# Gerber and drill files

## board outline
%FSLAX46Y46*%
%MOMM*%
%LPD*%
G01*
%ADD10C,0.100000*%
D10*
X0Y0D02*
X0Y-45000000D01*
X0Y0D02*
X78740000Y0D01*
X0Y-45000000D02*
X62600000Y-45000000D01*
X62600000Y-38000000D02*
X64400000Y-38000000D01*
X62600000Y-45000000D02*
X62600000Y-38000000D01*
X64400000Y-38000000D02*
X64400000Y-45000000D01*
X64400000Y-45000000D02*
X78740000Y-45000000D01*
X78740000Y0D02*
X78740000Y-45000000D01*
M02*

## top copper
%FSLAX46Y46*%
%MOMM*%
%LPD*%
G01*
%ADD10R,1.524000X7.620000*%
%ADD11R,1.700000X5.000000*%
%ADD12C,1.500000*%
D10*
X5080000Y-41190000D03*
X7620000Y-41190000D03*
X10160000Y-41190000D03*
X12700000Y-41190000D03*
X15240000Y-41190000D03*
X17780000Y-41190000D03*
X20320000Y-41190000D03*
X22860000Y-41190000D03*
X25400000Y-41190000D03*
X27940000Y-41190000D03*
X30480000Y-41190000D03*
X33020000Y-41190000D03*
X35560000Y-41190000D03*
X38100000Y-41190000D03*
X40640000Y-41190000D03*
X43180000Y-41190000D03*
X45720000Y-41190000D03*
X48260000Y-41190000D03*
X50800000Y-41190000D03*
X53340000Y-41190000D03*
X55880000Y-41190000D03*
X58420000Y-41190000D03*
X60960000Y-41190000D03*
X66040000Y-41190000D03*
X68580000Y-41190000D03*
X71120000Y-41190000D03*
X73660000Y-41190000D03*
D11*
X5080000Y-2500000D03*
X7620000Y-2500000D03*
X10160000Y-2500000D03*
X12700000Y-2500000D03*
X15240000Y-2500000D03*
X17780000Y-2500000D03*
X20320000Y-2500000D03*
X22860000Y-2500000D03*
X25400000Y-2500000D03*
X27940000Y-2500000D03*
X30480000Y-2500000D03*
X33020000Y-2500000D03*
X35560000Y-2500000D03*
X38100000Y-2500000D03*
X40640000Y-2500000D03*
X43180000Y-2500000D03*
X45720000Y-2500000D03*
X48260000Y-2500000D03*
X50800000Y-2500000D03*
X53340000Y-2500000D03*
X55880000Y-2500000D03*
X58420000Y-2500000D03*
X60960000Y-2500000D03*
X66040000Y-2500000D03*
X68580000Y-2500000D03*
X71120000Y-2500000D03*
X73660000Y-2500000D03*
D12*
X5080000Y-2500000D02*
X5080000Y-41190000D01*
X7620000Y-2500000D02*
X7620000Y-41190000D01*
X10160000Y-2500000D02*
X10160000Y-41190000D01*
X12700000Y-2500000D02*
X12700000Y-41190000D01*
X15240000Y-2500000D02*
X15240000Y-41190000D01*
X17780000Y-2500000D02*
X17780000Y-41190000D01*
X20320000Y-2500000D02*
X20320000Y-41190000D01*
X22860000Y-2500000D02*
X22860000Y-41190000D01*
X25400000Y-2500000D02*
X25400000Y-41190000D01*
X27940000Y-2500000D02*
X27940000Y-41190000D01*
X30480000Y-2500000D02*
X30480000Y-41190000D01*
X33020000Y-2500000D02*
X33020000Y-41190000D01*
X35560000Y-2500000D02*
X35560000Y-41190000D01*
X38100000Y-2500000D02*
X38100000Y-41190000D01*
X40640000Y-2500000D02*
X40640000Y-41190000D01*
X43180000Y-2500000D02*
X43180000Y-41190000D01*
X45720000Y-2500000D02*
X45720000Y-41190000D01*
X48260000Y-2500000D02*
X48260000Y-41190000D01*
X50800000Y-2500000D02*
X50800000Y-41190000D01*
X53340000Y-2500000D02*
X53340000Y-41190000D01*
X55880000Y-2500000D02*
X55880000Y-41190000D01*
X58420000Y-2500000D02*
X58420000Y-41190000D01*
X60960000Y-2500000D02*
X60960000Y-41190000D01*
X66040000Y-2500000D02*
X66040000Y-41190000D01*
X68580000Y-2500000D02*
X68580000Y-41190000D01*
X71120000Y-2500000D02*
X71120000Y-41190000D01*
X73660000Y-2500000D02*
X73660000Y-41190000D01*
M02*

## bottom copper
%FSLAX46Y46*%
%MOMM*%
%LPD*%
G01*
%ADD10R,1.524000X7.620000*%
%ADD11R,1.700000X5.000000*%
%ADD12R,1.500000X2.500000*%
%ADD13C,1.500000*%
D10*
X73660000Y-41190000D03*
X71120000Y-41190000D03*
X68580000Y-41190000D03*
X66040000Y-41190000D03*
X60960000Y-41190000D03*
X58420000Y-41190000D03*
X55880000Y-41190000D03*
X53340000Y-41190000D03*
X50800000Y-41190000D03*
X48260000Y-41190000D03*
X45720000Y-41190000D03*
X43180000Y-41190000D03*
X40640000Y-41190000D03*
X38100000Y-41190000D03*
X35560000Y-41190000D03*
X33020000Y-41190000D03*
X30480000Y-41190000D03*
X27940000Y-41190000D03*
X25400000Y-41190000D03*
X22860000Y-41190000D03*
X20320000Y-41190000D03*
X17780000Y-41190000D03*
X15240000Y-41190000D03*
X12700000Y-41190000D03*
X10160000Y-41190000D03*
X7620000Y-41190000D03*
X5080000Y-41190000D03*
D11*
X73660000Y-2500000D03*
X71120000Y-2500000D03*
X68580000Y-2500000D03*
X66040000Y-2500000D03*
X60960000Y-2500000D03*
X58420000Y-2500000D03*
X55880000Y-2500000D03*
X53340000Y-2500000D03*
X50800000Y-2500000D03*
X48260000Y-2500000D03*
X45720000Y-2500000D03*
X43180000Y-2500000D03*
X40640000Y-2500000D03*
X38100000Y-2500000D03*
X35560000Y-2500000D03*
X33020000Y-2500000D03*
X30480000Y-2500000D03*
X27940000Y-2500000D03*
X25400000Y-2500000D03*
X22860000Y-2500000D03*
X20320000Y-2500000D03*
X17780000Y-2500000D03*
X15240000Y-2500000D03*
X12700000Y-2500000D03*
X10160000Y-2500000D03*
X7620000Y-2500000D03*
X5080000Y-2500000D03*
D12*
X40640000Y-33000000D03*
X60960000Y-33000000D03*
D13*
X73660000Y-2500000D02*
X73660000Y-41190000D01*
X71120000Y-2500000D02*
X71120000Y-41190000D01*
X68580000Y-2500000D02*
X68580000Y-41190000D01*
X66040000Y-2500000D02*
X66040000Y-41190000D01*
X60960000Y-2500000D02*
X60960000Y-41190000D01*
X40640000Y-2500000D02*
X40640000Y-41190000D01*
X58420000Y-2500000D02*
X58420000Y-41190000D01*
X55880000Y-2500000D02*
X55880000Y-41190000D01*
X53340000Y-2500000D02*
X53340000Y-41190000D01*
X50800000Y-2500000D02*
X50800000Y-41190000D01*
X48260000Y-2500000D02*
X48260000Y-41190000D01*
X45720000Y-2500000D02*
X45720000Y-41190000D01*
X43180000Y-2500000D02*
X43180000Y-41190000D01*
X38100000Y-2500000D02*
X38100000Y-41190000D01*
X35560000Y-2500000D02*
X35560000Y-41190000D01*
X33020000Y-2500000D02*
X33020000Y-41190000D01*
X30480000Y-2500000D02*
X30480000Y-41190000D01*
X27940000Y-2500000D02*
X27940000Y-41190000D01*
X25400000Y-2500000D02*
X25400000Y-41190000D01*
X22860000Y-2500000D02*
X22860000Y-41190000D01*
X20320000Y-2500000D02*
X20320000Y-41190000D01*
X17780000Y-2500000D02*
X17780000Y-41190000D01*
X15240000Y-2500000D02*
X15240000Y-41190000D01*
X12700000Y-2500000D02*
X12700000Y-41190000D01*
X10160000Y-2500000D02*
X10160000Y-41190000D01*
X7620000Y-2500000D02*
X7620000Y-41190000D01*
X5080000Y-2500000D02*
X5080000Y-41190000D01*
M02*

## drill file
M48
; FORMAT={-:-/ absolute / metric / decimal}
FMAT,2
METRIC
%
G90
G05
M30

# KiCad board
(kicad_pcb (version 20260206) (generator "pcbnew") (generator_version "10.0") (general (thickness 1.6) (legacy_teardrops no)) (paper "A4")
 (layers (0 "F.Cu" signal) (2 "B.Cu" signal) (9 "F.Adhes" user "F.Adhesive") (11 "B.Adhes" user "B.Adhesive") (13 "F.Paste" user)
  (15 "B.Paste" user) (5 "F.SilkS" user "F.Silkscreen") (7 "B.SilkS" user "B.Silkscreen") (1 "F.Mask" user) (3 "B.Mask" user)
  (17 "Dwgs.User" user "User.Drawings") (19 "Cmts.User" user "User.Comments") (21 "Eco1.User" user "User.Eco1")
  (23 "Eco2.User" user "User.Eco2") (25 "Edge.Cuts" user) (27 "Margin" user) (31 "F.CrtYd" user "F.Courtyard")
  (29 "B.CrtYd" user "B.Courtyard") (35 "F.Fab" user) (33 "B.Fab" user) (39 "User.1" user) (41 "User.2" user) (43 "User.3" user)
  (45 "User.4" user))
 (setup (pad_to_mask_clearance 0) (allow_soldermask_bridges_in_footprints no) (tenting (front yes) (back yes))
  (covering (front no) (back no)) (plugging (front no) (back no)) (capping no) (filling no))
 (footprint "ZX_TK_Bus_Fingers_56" (layer "F.Cu") (at 39.37 41.19 180)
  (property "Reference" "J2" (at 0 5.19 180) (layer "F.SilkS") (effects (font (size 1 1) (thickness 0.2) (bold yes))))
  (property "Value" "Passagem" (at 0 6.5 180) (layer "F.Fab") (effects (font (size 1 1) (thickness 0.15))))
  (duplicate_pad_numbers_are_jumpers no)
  (pad "1" smd rect (at -34.29 0 180) (size 1.524 7.62) (layers "B.Cu" "B.Mask") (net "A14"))
  (pad "2" smd rect (at -31.75 0 180) (size 1.524 7.62) (layers "B.Cu" "B.Mask") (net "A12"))
  (pad "3" smd rect (at -29.21 0 180) (size 1.524 7.62) (layers "B.Cu" "B.Mask") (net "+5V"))
  (pad "4" smd rect (at -26.67 0 180) (size 1.524 7.62) (layers "B.Cu" "B.Mask") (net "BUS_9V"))
  (pad "6" smd rect (at -21.59 0 180) (size 1.524 7.62) (layers "B.Cu" "B.Mask") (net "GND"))
  (pad "7" smd rect (at -19.05 0 180) (size 1.524 7.62) (layers "B.Cu" "B.Mask") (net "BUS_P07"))
  (pad "8" smd rect (at -16.51 0 180) (size 1.524 7.62) (layers "B.Cu" "B.Mask") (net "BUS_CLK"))
  (pad "9" smd rect (at -13.97 0 180) (size 1.524 7.62) (layers "B.Cu" "B.Mask") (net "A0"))
  (pad "10" smd rect (at -11.43 0 180) (size 1.524 7.62) (layers "B.Cu" "B.Mask") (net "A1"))
  (pad "11" smd rect (at -8.89 0 180) (size 1.524 7.62) (layers "B.Cu" "B.Mask") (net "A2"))
  (pad "12" smd rect (at -6.35 0 180) (size 1.524 7.62) (layers "B.Cu" "B.Mask") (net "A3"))
  (pad "13" smd rect (at -3.81 0 180) (size 1.524 7.62) (layers "B.Cu" "B.Mask") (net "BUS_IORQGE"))
  (pad "14" smd rect (at -1.27 0 180) (size 1.524 7.62) (layers "B.Cu" "B.Mask") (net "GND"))
  (pad "15" smd rect (at 1.27 0 180) (size 1.524 7.62) (layers "B.Cu" "B.Mask") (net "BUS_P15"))
  (pad "16" smd rect (at 3.81 0 180) (size 1.524 7.62) (layers "B.Cu" "B.Mask") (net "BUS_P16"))
  (pad "17" smd rect (at 6.35 0 180) (size 1.524 7.62) (layers "B.Cu" "B.Mask") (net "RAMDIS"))
  (pad "18" smd rect (at 8.89 0 180) (size 1.524 7.62) (layers "B.Cu" "B.Mask") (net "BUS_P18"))
  (pad "19" smd rect (at 11.43 0 180) (size 1.524 7.62) (layers "B.Cu" "B.Mask") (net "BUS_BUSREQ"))
  (pad "20" smd rect (at 13.97 0 180) (size 1.524 7.62) (layers "B.Cu" "B.Mask") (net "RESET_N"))
  (pad "21" smd rect (at 16.51 0 180) (size 1.524 7.62) (layers "B.Cu" "B.Mask") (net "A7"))
  (pad "22" smd rect (at 19.05 0 180) (size 1.524 7.62) (layers "B.Cu" "B.Mask") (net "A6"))
  (pad "23" smd rect (at 21.59 0 180) (size 1.524 7.62) (layers "B.Cu" "B.Mask") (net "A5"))
  (pad "24" smd rect (at 24.13 0 180) (size 1.524 7.62) (layers "B.Cu" "B.Mask") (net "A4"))
  (pad "25" smd rect (at 26.67 0 180) (size 1.524 7.62) (layers "B.Cu" "B.Mask") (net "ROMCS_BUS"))
  (pad "26" smd rect (at 29.21 0 180) (size 1.524 7.62) (layers "B.Cu" "B.Mask") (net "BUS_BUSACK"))
  (pad "27" smd rect (at 31.75 0 180) (size 1.524 7.62) (layers "B.Cu" "B.Mask") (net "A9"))
  (pad "28" smd rect (at 34.29 0 180) (size 1.524 7.62) (layers "B.Cu" "B.Mask") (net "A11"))
  (pad "29" smd rect (at 34.29 0 180) (size 1.524 7.62) (layers "F.Cu" "F.Mask") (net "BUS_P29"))
  (pad "30" smd rect (at 31.75 0 180) (size 1.524 7.62) (layers "F.Cu" "F.Mask") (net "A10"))
  (pad "31" smd rect (at 29.21 0 180) (size 1.524 7.62) (layers "F.Cu" "F.Mask") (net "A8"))
  (pad "32" smd rect (at 26.67 0 180) (size 1.524 7.62) (layers "F.Cu" "F.Mask") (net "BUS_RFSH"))
  (pad "33" smd rect (at 24.13 0 180) (size 1.524 7.62) (layers "F.Cu" "F.Mask") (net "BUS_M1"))
  (pad "34" smd rect (at 21.59 0 180) (size 1.524 7.62) (layers "F.Cu" "F.Mask") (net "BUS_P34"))
  (pad "35" smd rect (at 19.05 0 180) (size 1.524 7.62) (layers "F.Cu" "F.Mask") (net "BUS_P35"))
  (pad "36" smd rect (at 16.51 0 180) (size 1.524 7.62) (layers "F.Cu" "F.Mask") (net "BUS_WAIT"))
  (pad "37" smd rect (at 13.97 0 180) (size 1.524 7.62) (layers "F.Cu" "F.Mask") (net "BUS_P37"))
  (pad "38" smd rect (at 11.43 0 180) (size 1.524 7.62) (layers "F.Cu" "F.Mask") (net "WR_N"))
  (pad "39" smd rect (at 8.89 0 180) (size 1.524 7.62) (layers "F.Cu" "F.Mask") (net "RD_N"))
  (pad "40" smd rect (at 6.35 0 180) (size 1.524 7.62) (layers "F.Cu" "F.Mask") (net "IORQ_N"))
  (pad "41" smd rect (at 3.81 0 180) (size 1.524 7.62) (layers "F.Cu" "F.Mask") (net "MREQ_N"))
  (pad "42" smd rect (at 1.27 0 180) (size 1.524 7.62) (layers "F.Cu" "F.Mask") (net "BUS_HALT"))
  (pad "43" smd rect (at -1.27 0 180) (size 1.524 7.62) (layers "F.Cu" "F.Mask") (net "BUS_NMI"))
  (pad "44" smd rect (at -3.81 0 180) (size 1.524 7.62) (layers "F.Cu" "F.Mask") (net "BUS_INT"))
  (pad "45" smd rect (at -6.35 0 180) (size 1.524 7.62) (layers "F.Cu" "F.Mask") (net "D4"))
  (pad "46" smd rect (at -8.89 0 180) (size 1.524 7.62) (layers "F.Cu" "F.Mask") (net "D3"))
  (pad "47" smd rect (at -11.43 0 180) (size 1.524 7.62) (layers "F.Cu" "F.Mask") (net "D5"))
  (pad "48" smd rect (at -13.97 0 180) (size 1.524 7.62) (layers "F.Cu" "F.Mask") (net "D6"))
  (pad "49" smd rect (at -16.51 0 180) (size 1.524 7.62) (layers "F.Cu" "F.Mask") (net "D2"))
  (pad "50" smd rect (at -19.05 0 180) (size 1.524 7.62) (layers "F.Cu" "F.Mask") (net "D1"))
  (pad "51" smd rect (at -21.59 0 180) (size 1.524 7.62) (layers "F.Cu" "F.Mask") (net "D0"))
  (pad "53" smd rect (at -26.67 0 180) (size 1.524 7.62) (layers "F.Cu" "F.Mask") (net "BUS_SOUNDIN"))
  (pad "54" smd rect (at -29.21 0 180) (size 1.524 7.62) (layers "F.Cu" "F.Mask") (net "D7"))
  (pad "55" smd rect (at -31.75 0 180) (size 1.524 7.62) (layers "F.Cu" "F.Mask") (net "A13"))
  (pad "56" smd rect (at -34.29 0 180) (size 1.524 7.62) (layers "F.Cu" "F.Mask") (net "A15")))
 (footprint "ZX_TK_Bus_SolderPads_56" (layer "F.Cu") (at 39.37 2.5 180)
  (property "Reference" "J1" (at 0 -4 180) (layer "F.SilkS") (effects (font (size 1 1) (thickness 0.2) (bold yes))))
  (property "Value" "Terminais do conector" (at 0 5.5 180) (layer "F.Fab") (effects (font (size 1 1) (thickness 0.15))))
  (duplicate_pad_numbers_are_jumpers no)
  (pad "1" smd rect (at -34.29 0 180) (size 1.7 5) (layers "B.Cu" "B.Mask" "B.Paste") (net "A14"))
  (pad "2" smd rect (at -31.75 0 180) (size 1.7 5) (layers "B.Cu" "B.Mask" "B.Paste") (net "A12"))
  (pad "3" smd rect (at -29.21 0 180) (size 1.7 5) (layers "B.Cu" "B.Mask" "B.Paste") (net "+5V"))
  (pad "4" smd rect (at -26.67 0 180) (size 1.7 5) (layers "B.Cu" "B.Mask" "B.Paste") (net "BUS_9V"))
  (pad "6" smd rect (at -21.59 0 180) (size 1.7 5) (layers "B.Cu" "B.Mask" "B.Paste") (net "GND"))
  (pad "7" smd rect (at -19.05 0 180) (size 1.7 5) (layers "B.Cu" "B.Mask" "B.Paste") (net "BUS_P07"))
  (pad "8" smd rect (at -16.51 0 180) (size 1.7 5) (layers "B.Cu" "B.Mask" "B.Paste") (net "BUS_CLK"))
  (pad "9" smd rect (at -13.97 0 180) (size 1.7 5) (layers "B.Cu" "B.Mask" "B.Paste") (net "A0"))
  (pad "10" smd rect (at -11.43 0 180) (size 1.7 5) (layers "B.Cu" "B.Mask" "B.Paste") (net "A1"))
  (pad "11" smd rect (at -8.89 0 180) (size 1.7 5) (layers "B.Cu" "B.Mask" "B.Paste") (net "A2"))
  (pad "12" smd rect (at -6.35 0 180) (size 1.7 5) (layers "B.Cu" "B.Mask" "B.Paste") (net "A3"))
  (pad "13" smd rect (at -3.81 0 180) (size 1.7 5) (layers "B.Cu" "B.Mask" "B.Paste") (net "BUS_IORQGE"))
  (pad "14" smd rect (at -1.27 0 180) (size 1.7 5) (layers "B.Cu" "B.Mask" "B.Paste") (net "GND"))
  (pad "15" smd rect (at 1.27 0 180) (size 1.7 5) (layers "B.Cu" "B.Mask" "B.Paste") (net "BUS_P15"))
  (pad "16" smd rect (at 3.81 0 180) (size 1.7 5) (layers "B.Cu" "B.Mask" "B.Paste") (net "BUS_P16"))
  (pad "17" smd rect (at 6.35 0 180) (size 1.7 5) (layers "B.Cu" "B.Mask" "B.Paste") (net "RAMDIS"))
  (pad "18" smd rect (at 8.89 0 180) (size 1.7 5) (layers "B.Cu" "B.Mask" "B.Paste") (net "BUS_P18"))
  (pad "19" smd rect (at 11.43 0 180) (size 1.7 5) (layers "B.Cu" "B.Mask" "B.Paste") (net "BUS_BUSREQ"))
  (pad "20" smd rect (at 13.97 0 180) (size 1.7 5) (layers "B.Cu" "B.Mask" "B.Paste") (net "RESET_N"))
  (pad "21" smd rect (at 16.51 0 180) (size 1.7 5) (layers "B.Cu" "B.Mask" "B.Paste") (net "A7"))
  (pad "22" smd rect (at 19.05 0 180) (size 1.7 5) (layers "B.Cu" "B.Mask" "B.Paste") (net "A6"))
  (pad "23" smd rect (at 21.59 0 180) (size 1.7 5) (layers "B.Cu" "B.Mask" "B.Paste") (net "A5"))
  (pad "24" smd rect (at 24.13 0 180) (size 1.7 5) (layers "B.Cu" "B.Mask" "B.Paste") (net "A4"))
  (pad "25" smd rect (at 26.67 0 180) (size 1.7 5) (layers "B.Cu" "B.Mask" "B.Paste") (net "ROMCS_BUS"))
  (pad "26" smd rect (at 29.21 0 180) (size 1.7 5) (layers "B.Cu" "B.Mask" "B.Paste") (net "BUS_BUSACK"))
  (pad "27" smd rect (at 31.75 0 180) (size 1.7 5) (layers "B.Cu" "B.Mask" "B.Paste") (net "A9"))
  (pad "28" smd rect (at 34.29 0 180) (size 1.7 5) (layers "B.Cu" "B.Mask" "B.Paste") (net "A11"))
  (pad "29" smd rect (at 34.29 0 180) (size 1.7 5) (layers "F.Cu" "F.Mask" "F.Paste") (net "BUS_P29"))
  (pad "30" smd rect (at 31.75 0 180) (size 1.7 5) (layers "F.Cu" "F.Mask" "F.Paste") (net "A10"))
  (pad "31" smd rect (at 29.21 0 180) (size 1.7 5) (layers "F.Cu" "F.Mask" "F.Paste") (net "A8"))
  (pad "32" smd rect (at 26.67 0 180) (size 1.7 5) (layers "F.Cu" "F.Mask" "F.Paste") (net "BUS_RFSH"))
  (pad "33" smd rect (at 24.13 0 180) (size 1.7 5) (layers "F.Cu" "F.Mask" "F.Paste") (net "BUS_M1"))
  (pad "34" smd rect (at 21.59 0 180) (size 1.7 5) (layers "F.Cu" "F.Mask" "F.Paste") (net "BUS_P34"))
  (pad "35" smd rect (at 19.05 0 180) (size 1.7 5) (layers "F.Cu" "F.Mask" "F.Paste") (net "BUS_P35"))
  (pad "36" smd rect (at 16.51 0 180) (size 1.7 5) (layers "F.Cu" "F.Mask" "F.Paste") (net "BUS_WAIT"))
  (pad "37" smd rect (at 13.97 0 180) (size 1.7 5) (layers "F.Cu" "F.Mask" "F.Paste") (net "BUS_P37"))
  (pad "38" smd rect (at 11.43 0 180) (size 1.7 5) (layers "F.Cu" "F.Mask" "F.Paste") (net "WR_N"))
  (pad "39" smd rect (at 8.89 0 180) (size 1.7 5) (layers "F.Cu" "F.Mask" "F.Paste") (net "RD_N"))
  (pad "40" smd rect (at 6.35 0 180) (size 1.7 5) (layers "F.Cu" "F.Mask" "F.Paste") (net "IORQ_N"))
  (pad "41" smd rect (at 3.81 0 180) (size 1.7 5) (layers "F.Cu" "F.Mask" "F.Paste") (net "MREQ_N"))
  (pad "42" smd rect (at 1.27 0 180) (size 1.7 5) (layers "F.Cu" "F.Mask" "F.Paste") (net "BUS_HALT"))
  (pad "43" smd rect (at -1.27 0 180) (size 1.7 5) (layers "F.Cu" "F.Mask" "F.Paste") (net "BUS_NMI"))
  (pad "44" smd rect (at -3.81 0 180) (size 1.7 5) (layers "F.Cu" "F.Mask" "F.Paste") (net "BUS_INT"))
  (pad "45" smd rect (at -6.35 0 180) (size 1.7 5) (layers "F.Cu" "F.Mask" "F.Paste") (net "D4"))
  (pad "46" smd rect (at -8.89 0 180) (size 1.7 5) (layers "F.Cu" "F.Mask" "F.Paste") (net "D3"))
  (pad "47" smd rect (at -11.43 0 180) (size 1.7 5) (layers "F.Cu" "F.Mask" "F.Paste") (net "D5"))
  (pad "48" smd rect (at -13.97 0 180) (size 1.7 5) (layers "F.Cu" "F.Mask" "F.Paste") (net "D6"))
  (pad "49" smd rect (at -16.51 0 180) (size 1.7 5) (layers "F.Cu" "F.Mask" "F.Paste") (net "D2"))
  (pad "50" smd rect (at -19.05 0 180) (size 1.7 5) (layers "F.Cu" "F.Mask" "F.Paste") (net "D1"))
  (pad "51" smd rect (at -21.59 0 180) (size 1.7 5) (layers "F.Cu" "F.Mask" "F.Paste") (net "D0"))
  (pad "53" smd rect (at -26.67 0 180) (size 1.7 5) (layers "F.Cu" "F.Mask" "F.Paste") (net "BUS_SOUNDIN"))
  (pad "54" smd rect (at -29.21 0 180) (size 1.7 5) (layers "F.Cu" "F.Mask" "F.Paste") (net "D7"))
  (pad "55" smd rect (at -31.75 0 180) (size 1.7 5) (layers "F.Cu" "F.Mask" "F.Paste") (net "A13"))
  (pad "56" smd rect (at -34.29 0 180) (size 1.7 5) (layers "F.Cu" "F.Mask" "F.Paste") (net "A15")))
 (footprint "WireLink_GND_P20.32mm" (layer "F.Cu") (at 50.8 33)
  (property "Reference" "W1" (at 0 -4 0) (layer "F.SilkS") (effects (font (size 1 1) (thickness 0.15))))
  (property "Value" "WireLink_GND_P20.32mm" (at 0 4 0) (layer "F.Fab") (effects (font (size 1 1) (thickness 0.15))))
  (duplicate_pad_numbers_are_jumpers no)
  (pad "1" smd rect (at -10.16 0) (size 1.5 2.5) (layers "B.Cu" "B.Mask" "B.Paste") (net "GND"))
  (pad "1" smd rect (at 10.16 0) (size 1.5 2.5) (layers "B.Cu" "B.Mask" "B.Paste") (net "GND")))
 (gr_line (start 0 0) (end 0 45) (stroke (width 0.1) (type default)) (layer "Edge.Cuts"))
 (gr_line (start 0 0) (end 78.74 0) (stroke (width 0.1) (type default)) (layer "Edge.Cuts"))
 (gr_line (start 0 45) (end 62.6 45) (stroke (width 0.1) (type default)) (layer "Edge.Cuts"))
 (gr_line (start 62.6 38) (end 64.4 38) (stroke (width 0.1) (type default)) (layer "Edge.Cuts"))
 (gr_line (start 62.6 45) (end 62.6 38) (stroke (width 0.1) (type default)) (layer "Edge.Cuts"))
 (gr_line (start 64.4 38) (end 64.4 45) (stroke (width 0.1) (type default)) (layer "Edge.Cuts"))
 (gr_line (start 64.4 45) (end 78.74 45) (stroke (width 0.1) (type default)) (layer "Edge.Cuts"))
 (gr_line (start 78.74 0) (end 78.74 45) (stroke (width 0.1) (type default)) (layer "Edge.Cuts"))
 (segment (start 73.66 2.5) (end 73.66 41.19) (width 1.5) (layer "B.Cu") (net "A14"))
 (segment (start 71.12 2.5) (end 71.12 41.19) (width 1.5) (layer "B.Cu") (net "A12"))
 (segment (start 68.58 2.5) (end 68.58 41.19) (width 1.5) (layer "B.Cu") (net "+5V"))
 (segment (start 66.04 2.5) (end 66.04 41.19) (width 1.5) (layer "B.Cu") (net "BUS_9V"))
 (segment (start 60.96 2.5) (end 60.96 41.19) (width 1.5) (layer "B.Cu") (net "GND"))
 (segment (start 40.64 2.5) (end 40.64 41.19) (width 1.5) (layer "B.Cu") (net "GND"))
 (segment (start 58.42 2.5) (end 58.42 41.19) (width 1.5) (layer "B.Cu") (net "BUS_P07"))
 (segment (start 55.88 2.5) (end 55.88 41.19) (width 1.5) (layer "B.Cu") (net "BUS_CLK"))
 (segment (start 53.34 2.5) (end 53.34 41.19) (width 1.5) (layer "B.Cu") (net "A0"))
 (segment (start 50.8 2.5) (end 50.8 41.19) (width 1.5) (layer "B.Cu") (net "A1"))
 (segment (start 48.26 2.5) (end 48.26 41.19) (width 1.5) (layer "B.Cu") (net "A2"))
 (segment (start 45.72 2.5) (end 45.72 41.19) (width 1.5) (layer "B.Cu") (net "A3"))
 (segment (start 43.18 2.5) (end 43.18 41.19) (width 1.5) (layer "B.Cu") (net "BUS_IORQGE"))
 (segment (start 38.1 2.5) (end 38.1 41.19) (width 1.5) (layer "B.Cu") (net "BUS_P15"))
 (segment (start 35.56 2.5) (end 35.56 41.19) (width 1.5) (layer "B.Cu") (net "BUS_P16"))
 (segment (start 33.02 2.5) (end 33.02 41.19) (width 1.5) (layer "B.Cu") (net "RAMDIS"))
 (segment (start 30.48 2.5) (end 30.48 41.19) (width 1.5) (layer "B.Cu") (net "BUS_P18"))
 (segment (start 27.94 2.5) (end 27.94 41.19) (width 1.5) (layer "B.Cu") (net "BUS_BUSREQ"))
 (segment (start 25.4 2.5) (end 25.4 41.19) (width 1.5) (layer "B.Cu") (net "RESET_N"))
 (segment (start 22.86 2.5) (end 22.86 41.19) (width 1.5) (layer "B.Cu") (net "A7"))
 (segment (start 20.32 2.5) (end 20.32 41.19) (width 1.5) (layer "B.Cu") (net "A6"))
 (segment (start 17.78 2.5) (end 17.78 41.19) (width 1.5) (layer "B.Cu") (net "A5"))
 (segment (start 15.24 2.5) (end 15.24 41.19) (width 1.5) (layer "B.Cu") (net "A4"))
 (segment (start 12.7 2.5) (end 12.7 41.19) (width 1.5) (layer "B.Cu") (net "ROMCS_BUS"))
 (segment (start 10.16 2.5) (end 10.16 41.19) (width 1.5) (layer "B.Cu") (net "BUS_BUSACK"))
 (segment (start 7.62 2.5) (end 7.62 41.19) (width 1.5) (layer "B.Cu") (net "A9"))
 (segment (start 5.08 2.5) (end 5.08 41.19) (width 1.5) (layer "B.Cu") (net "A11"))
 (segment (start 5.08 2.5) (end 5.08 41.19) (width 1.5) (layer "F.Cu") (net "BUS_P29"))
 (segment (start 7.62 2.5) (end 7.62 41.19) (width 1.5) (layer "F.Cu") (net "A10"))
 (segment (start 10.16 2.5) (end 10.16 41.19) (width 1.5) (layer "F.Cu") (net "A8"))
 (segment (start 12.7 2.5) (end 12.7 41.19) (width 1.5) (layer "F.Cu") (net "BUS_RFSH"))
 (segment (start 15.24 2.5) (end 15.24 41.19) (width 1.5) (layer "F.Cu") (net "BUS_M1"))
 (segment (start 17.78 2.5) (end 17.78 41.19) (width 1.5) (layer "F.Cu") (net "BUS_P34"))
 (segment (start 20.32 2.5) (end 20.32 41.19) (width 1.5) (layer "F.Cu") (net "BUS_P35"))
 (segment (start 22.86 2.5) (end 22.86 41.19) (width 1.5) (layer "F.Cu") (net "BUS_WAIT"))
 (segment (start 25.4 2.5) (end 25.4 41.19) (width 1.5) (layer "F.Cu") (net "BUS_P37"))
 (segment (start 27.94 2.5) (end 27.94 41.19) (width 1.5) (layer "F.Cu") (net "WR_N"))
 (segment (start 30.48 2.5) (end 30.48 41.19) (width 1.5) (layer "F.Cu") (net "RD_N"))
 (segment (start 33.02 2.5) (end 33.02 41.19) (width 1.5) (layer "F.Cu") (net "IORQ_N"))
 (segment (start 35.56 2.5) (end 35.56 41.19) (width 1.5) (layer "F.Cu") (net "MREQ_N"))
 (segment (start 38.1 2.5) (end 38.1 41.19) (width 1.5) (layer "F.Cu") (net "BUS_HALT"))
 (segment (start 40.64 2.5) (end 40.64 41.19) (width 1.5) (layer "F.Cu") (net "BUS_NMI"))
 (segment (start 43.18 2.5) (end 43.18 41.19) (width 1.5) (layer "F.Cu") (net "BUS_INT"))
 (segment (start 45.72 2.5) (end 45.72 41.19) (width 1.5) (layer "F.Cu") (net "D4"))
 (segment (start 48.26 2.5) (end 48.26 41.19) (width 1.5) (layer "F.Cu") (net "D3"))
 (segment (start 50.8 2.5) (end 50.8 41.19) (width 1.5) (layer "F.Cu") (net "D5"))
 (segment (start 53.34 2.5) (end 53.34 41.19) (width 1.5) (layer "F.Cu") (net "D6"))
 (segment (start 55.88 2.5) (end 55.88 41.19) (width 1.5) (layer "F.Cu") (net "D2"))
 (segment (start 58.42 2.5) (end 58.42 41.19) (width 1.5) (layer "F.Cu") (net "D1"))
 (segment (start 60.96 2.5) (end 60.96 41.19) (width 1.5) (layer "F.Cu") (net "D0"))
 (segment (start 66.04 2.5) (end 66.04 41.19) (width 1.5) (layer "F.Cu") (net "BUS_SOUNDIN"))
 (segment (start 68.58 2.5) (end 68.58 41.19) (width 1.5) (layer "F.Cu") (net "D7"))
 (segment (start 71.12 2.5) (end 71.12 41.19) (width 1.5) (layer "F.Cu") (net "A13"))
 (segment (start 73.66 2.5) (end 73.66 41.19) (width 1.5) (layer "F.Cu") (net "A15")))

